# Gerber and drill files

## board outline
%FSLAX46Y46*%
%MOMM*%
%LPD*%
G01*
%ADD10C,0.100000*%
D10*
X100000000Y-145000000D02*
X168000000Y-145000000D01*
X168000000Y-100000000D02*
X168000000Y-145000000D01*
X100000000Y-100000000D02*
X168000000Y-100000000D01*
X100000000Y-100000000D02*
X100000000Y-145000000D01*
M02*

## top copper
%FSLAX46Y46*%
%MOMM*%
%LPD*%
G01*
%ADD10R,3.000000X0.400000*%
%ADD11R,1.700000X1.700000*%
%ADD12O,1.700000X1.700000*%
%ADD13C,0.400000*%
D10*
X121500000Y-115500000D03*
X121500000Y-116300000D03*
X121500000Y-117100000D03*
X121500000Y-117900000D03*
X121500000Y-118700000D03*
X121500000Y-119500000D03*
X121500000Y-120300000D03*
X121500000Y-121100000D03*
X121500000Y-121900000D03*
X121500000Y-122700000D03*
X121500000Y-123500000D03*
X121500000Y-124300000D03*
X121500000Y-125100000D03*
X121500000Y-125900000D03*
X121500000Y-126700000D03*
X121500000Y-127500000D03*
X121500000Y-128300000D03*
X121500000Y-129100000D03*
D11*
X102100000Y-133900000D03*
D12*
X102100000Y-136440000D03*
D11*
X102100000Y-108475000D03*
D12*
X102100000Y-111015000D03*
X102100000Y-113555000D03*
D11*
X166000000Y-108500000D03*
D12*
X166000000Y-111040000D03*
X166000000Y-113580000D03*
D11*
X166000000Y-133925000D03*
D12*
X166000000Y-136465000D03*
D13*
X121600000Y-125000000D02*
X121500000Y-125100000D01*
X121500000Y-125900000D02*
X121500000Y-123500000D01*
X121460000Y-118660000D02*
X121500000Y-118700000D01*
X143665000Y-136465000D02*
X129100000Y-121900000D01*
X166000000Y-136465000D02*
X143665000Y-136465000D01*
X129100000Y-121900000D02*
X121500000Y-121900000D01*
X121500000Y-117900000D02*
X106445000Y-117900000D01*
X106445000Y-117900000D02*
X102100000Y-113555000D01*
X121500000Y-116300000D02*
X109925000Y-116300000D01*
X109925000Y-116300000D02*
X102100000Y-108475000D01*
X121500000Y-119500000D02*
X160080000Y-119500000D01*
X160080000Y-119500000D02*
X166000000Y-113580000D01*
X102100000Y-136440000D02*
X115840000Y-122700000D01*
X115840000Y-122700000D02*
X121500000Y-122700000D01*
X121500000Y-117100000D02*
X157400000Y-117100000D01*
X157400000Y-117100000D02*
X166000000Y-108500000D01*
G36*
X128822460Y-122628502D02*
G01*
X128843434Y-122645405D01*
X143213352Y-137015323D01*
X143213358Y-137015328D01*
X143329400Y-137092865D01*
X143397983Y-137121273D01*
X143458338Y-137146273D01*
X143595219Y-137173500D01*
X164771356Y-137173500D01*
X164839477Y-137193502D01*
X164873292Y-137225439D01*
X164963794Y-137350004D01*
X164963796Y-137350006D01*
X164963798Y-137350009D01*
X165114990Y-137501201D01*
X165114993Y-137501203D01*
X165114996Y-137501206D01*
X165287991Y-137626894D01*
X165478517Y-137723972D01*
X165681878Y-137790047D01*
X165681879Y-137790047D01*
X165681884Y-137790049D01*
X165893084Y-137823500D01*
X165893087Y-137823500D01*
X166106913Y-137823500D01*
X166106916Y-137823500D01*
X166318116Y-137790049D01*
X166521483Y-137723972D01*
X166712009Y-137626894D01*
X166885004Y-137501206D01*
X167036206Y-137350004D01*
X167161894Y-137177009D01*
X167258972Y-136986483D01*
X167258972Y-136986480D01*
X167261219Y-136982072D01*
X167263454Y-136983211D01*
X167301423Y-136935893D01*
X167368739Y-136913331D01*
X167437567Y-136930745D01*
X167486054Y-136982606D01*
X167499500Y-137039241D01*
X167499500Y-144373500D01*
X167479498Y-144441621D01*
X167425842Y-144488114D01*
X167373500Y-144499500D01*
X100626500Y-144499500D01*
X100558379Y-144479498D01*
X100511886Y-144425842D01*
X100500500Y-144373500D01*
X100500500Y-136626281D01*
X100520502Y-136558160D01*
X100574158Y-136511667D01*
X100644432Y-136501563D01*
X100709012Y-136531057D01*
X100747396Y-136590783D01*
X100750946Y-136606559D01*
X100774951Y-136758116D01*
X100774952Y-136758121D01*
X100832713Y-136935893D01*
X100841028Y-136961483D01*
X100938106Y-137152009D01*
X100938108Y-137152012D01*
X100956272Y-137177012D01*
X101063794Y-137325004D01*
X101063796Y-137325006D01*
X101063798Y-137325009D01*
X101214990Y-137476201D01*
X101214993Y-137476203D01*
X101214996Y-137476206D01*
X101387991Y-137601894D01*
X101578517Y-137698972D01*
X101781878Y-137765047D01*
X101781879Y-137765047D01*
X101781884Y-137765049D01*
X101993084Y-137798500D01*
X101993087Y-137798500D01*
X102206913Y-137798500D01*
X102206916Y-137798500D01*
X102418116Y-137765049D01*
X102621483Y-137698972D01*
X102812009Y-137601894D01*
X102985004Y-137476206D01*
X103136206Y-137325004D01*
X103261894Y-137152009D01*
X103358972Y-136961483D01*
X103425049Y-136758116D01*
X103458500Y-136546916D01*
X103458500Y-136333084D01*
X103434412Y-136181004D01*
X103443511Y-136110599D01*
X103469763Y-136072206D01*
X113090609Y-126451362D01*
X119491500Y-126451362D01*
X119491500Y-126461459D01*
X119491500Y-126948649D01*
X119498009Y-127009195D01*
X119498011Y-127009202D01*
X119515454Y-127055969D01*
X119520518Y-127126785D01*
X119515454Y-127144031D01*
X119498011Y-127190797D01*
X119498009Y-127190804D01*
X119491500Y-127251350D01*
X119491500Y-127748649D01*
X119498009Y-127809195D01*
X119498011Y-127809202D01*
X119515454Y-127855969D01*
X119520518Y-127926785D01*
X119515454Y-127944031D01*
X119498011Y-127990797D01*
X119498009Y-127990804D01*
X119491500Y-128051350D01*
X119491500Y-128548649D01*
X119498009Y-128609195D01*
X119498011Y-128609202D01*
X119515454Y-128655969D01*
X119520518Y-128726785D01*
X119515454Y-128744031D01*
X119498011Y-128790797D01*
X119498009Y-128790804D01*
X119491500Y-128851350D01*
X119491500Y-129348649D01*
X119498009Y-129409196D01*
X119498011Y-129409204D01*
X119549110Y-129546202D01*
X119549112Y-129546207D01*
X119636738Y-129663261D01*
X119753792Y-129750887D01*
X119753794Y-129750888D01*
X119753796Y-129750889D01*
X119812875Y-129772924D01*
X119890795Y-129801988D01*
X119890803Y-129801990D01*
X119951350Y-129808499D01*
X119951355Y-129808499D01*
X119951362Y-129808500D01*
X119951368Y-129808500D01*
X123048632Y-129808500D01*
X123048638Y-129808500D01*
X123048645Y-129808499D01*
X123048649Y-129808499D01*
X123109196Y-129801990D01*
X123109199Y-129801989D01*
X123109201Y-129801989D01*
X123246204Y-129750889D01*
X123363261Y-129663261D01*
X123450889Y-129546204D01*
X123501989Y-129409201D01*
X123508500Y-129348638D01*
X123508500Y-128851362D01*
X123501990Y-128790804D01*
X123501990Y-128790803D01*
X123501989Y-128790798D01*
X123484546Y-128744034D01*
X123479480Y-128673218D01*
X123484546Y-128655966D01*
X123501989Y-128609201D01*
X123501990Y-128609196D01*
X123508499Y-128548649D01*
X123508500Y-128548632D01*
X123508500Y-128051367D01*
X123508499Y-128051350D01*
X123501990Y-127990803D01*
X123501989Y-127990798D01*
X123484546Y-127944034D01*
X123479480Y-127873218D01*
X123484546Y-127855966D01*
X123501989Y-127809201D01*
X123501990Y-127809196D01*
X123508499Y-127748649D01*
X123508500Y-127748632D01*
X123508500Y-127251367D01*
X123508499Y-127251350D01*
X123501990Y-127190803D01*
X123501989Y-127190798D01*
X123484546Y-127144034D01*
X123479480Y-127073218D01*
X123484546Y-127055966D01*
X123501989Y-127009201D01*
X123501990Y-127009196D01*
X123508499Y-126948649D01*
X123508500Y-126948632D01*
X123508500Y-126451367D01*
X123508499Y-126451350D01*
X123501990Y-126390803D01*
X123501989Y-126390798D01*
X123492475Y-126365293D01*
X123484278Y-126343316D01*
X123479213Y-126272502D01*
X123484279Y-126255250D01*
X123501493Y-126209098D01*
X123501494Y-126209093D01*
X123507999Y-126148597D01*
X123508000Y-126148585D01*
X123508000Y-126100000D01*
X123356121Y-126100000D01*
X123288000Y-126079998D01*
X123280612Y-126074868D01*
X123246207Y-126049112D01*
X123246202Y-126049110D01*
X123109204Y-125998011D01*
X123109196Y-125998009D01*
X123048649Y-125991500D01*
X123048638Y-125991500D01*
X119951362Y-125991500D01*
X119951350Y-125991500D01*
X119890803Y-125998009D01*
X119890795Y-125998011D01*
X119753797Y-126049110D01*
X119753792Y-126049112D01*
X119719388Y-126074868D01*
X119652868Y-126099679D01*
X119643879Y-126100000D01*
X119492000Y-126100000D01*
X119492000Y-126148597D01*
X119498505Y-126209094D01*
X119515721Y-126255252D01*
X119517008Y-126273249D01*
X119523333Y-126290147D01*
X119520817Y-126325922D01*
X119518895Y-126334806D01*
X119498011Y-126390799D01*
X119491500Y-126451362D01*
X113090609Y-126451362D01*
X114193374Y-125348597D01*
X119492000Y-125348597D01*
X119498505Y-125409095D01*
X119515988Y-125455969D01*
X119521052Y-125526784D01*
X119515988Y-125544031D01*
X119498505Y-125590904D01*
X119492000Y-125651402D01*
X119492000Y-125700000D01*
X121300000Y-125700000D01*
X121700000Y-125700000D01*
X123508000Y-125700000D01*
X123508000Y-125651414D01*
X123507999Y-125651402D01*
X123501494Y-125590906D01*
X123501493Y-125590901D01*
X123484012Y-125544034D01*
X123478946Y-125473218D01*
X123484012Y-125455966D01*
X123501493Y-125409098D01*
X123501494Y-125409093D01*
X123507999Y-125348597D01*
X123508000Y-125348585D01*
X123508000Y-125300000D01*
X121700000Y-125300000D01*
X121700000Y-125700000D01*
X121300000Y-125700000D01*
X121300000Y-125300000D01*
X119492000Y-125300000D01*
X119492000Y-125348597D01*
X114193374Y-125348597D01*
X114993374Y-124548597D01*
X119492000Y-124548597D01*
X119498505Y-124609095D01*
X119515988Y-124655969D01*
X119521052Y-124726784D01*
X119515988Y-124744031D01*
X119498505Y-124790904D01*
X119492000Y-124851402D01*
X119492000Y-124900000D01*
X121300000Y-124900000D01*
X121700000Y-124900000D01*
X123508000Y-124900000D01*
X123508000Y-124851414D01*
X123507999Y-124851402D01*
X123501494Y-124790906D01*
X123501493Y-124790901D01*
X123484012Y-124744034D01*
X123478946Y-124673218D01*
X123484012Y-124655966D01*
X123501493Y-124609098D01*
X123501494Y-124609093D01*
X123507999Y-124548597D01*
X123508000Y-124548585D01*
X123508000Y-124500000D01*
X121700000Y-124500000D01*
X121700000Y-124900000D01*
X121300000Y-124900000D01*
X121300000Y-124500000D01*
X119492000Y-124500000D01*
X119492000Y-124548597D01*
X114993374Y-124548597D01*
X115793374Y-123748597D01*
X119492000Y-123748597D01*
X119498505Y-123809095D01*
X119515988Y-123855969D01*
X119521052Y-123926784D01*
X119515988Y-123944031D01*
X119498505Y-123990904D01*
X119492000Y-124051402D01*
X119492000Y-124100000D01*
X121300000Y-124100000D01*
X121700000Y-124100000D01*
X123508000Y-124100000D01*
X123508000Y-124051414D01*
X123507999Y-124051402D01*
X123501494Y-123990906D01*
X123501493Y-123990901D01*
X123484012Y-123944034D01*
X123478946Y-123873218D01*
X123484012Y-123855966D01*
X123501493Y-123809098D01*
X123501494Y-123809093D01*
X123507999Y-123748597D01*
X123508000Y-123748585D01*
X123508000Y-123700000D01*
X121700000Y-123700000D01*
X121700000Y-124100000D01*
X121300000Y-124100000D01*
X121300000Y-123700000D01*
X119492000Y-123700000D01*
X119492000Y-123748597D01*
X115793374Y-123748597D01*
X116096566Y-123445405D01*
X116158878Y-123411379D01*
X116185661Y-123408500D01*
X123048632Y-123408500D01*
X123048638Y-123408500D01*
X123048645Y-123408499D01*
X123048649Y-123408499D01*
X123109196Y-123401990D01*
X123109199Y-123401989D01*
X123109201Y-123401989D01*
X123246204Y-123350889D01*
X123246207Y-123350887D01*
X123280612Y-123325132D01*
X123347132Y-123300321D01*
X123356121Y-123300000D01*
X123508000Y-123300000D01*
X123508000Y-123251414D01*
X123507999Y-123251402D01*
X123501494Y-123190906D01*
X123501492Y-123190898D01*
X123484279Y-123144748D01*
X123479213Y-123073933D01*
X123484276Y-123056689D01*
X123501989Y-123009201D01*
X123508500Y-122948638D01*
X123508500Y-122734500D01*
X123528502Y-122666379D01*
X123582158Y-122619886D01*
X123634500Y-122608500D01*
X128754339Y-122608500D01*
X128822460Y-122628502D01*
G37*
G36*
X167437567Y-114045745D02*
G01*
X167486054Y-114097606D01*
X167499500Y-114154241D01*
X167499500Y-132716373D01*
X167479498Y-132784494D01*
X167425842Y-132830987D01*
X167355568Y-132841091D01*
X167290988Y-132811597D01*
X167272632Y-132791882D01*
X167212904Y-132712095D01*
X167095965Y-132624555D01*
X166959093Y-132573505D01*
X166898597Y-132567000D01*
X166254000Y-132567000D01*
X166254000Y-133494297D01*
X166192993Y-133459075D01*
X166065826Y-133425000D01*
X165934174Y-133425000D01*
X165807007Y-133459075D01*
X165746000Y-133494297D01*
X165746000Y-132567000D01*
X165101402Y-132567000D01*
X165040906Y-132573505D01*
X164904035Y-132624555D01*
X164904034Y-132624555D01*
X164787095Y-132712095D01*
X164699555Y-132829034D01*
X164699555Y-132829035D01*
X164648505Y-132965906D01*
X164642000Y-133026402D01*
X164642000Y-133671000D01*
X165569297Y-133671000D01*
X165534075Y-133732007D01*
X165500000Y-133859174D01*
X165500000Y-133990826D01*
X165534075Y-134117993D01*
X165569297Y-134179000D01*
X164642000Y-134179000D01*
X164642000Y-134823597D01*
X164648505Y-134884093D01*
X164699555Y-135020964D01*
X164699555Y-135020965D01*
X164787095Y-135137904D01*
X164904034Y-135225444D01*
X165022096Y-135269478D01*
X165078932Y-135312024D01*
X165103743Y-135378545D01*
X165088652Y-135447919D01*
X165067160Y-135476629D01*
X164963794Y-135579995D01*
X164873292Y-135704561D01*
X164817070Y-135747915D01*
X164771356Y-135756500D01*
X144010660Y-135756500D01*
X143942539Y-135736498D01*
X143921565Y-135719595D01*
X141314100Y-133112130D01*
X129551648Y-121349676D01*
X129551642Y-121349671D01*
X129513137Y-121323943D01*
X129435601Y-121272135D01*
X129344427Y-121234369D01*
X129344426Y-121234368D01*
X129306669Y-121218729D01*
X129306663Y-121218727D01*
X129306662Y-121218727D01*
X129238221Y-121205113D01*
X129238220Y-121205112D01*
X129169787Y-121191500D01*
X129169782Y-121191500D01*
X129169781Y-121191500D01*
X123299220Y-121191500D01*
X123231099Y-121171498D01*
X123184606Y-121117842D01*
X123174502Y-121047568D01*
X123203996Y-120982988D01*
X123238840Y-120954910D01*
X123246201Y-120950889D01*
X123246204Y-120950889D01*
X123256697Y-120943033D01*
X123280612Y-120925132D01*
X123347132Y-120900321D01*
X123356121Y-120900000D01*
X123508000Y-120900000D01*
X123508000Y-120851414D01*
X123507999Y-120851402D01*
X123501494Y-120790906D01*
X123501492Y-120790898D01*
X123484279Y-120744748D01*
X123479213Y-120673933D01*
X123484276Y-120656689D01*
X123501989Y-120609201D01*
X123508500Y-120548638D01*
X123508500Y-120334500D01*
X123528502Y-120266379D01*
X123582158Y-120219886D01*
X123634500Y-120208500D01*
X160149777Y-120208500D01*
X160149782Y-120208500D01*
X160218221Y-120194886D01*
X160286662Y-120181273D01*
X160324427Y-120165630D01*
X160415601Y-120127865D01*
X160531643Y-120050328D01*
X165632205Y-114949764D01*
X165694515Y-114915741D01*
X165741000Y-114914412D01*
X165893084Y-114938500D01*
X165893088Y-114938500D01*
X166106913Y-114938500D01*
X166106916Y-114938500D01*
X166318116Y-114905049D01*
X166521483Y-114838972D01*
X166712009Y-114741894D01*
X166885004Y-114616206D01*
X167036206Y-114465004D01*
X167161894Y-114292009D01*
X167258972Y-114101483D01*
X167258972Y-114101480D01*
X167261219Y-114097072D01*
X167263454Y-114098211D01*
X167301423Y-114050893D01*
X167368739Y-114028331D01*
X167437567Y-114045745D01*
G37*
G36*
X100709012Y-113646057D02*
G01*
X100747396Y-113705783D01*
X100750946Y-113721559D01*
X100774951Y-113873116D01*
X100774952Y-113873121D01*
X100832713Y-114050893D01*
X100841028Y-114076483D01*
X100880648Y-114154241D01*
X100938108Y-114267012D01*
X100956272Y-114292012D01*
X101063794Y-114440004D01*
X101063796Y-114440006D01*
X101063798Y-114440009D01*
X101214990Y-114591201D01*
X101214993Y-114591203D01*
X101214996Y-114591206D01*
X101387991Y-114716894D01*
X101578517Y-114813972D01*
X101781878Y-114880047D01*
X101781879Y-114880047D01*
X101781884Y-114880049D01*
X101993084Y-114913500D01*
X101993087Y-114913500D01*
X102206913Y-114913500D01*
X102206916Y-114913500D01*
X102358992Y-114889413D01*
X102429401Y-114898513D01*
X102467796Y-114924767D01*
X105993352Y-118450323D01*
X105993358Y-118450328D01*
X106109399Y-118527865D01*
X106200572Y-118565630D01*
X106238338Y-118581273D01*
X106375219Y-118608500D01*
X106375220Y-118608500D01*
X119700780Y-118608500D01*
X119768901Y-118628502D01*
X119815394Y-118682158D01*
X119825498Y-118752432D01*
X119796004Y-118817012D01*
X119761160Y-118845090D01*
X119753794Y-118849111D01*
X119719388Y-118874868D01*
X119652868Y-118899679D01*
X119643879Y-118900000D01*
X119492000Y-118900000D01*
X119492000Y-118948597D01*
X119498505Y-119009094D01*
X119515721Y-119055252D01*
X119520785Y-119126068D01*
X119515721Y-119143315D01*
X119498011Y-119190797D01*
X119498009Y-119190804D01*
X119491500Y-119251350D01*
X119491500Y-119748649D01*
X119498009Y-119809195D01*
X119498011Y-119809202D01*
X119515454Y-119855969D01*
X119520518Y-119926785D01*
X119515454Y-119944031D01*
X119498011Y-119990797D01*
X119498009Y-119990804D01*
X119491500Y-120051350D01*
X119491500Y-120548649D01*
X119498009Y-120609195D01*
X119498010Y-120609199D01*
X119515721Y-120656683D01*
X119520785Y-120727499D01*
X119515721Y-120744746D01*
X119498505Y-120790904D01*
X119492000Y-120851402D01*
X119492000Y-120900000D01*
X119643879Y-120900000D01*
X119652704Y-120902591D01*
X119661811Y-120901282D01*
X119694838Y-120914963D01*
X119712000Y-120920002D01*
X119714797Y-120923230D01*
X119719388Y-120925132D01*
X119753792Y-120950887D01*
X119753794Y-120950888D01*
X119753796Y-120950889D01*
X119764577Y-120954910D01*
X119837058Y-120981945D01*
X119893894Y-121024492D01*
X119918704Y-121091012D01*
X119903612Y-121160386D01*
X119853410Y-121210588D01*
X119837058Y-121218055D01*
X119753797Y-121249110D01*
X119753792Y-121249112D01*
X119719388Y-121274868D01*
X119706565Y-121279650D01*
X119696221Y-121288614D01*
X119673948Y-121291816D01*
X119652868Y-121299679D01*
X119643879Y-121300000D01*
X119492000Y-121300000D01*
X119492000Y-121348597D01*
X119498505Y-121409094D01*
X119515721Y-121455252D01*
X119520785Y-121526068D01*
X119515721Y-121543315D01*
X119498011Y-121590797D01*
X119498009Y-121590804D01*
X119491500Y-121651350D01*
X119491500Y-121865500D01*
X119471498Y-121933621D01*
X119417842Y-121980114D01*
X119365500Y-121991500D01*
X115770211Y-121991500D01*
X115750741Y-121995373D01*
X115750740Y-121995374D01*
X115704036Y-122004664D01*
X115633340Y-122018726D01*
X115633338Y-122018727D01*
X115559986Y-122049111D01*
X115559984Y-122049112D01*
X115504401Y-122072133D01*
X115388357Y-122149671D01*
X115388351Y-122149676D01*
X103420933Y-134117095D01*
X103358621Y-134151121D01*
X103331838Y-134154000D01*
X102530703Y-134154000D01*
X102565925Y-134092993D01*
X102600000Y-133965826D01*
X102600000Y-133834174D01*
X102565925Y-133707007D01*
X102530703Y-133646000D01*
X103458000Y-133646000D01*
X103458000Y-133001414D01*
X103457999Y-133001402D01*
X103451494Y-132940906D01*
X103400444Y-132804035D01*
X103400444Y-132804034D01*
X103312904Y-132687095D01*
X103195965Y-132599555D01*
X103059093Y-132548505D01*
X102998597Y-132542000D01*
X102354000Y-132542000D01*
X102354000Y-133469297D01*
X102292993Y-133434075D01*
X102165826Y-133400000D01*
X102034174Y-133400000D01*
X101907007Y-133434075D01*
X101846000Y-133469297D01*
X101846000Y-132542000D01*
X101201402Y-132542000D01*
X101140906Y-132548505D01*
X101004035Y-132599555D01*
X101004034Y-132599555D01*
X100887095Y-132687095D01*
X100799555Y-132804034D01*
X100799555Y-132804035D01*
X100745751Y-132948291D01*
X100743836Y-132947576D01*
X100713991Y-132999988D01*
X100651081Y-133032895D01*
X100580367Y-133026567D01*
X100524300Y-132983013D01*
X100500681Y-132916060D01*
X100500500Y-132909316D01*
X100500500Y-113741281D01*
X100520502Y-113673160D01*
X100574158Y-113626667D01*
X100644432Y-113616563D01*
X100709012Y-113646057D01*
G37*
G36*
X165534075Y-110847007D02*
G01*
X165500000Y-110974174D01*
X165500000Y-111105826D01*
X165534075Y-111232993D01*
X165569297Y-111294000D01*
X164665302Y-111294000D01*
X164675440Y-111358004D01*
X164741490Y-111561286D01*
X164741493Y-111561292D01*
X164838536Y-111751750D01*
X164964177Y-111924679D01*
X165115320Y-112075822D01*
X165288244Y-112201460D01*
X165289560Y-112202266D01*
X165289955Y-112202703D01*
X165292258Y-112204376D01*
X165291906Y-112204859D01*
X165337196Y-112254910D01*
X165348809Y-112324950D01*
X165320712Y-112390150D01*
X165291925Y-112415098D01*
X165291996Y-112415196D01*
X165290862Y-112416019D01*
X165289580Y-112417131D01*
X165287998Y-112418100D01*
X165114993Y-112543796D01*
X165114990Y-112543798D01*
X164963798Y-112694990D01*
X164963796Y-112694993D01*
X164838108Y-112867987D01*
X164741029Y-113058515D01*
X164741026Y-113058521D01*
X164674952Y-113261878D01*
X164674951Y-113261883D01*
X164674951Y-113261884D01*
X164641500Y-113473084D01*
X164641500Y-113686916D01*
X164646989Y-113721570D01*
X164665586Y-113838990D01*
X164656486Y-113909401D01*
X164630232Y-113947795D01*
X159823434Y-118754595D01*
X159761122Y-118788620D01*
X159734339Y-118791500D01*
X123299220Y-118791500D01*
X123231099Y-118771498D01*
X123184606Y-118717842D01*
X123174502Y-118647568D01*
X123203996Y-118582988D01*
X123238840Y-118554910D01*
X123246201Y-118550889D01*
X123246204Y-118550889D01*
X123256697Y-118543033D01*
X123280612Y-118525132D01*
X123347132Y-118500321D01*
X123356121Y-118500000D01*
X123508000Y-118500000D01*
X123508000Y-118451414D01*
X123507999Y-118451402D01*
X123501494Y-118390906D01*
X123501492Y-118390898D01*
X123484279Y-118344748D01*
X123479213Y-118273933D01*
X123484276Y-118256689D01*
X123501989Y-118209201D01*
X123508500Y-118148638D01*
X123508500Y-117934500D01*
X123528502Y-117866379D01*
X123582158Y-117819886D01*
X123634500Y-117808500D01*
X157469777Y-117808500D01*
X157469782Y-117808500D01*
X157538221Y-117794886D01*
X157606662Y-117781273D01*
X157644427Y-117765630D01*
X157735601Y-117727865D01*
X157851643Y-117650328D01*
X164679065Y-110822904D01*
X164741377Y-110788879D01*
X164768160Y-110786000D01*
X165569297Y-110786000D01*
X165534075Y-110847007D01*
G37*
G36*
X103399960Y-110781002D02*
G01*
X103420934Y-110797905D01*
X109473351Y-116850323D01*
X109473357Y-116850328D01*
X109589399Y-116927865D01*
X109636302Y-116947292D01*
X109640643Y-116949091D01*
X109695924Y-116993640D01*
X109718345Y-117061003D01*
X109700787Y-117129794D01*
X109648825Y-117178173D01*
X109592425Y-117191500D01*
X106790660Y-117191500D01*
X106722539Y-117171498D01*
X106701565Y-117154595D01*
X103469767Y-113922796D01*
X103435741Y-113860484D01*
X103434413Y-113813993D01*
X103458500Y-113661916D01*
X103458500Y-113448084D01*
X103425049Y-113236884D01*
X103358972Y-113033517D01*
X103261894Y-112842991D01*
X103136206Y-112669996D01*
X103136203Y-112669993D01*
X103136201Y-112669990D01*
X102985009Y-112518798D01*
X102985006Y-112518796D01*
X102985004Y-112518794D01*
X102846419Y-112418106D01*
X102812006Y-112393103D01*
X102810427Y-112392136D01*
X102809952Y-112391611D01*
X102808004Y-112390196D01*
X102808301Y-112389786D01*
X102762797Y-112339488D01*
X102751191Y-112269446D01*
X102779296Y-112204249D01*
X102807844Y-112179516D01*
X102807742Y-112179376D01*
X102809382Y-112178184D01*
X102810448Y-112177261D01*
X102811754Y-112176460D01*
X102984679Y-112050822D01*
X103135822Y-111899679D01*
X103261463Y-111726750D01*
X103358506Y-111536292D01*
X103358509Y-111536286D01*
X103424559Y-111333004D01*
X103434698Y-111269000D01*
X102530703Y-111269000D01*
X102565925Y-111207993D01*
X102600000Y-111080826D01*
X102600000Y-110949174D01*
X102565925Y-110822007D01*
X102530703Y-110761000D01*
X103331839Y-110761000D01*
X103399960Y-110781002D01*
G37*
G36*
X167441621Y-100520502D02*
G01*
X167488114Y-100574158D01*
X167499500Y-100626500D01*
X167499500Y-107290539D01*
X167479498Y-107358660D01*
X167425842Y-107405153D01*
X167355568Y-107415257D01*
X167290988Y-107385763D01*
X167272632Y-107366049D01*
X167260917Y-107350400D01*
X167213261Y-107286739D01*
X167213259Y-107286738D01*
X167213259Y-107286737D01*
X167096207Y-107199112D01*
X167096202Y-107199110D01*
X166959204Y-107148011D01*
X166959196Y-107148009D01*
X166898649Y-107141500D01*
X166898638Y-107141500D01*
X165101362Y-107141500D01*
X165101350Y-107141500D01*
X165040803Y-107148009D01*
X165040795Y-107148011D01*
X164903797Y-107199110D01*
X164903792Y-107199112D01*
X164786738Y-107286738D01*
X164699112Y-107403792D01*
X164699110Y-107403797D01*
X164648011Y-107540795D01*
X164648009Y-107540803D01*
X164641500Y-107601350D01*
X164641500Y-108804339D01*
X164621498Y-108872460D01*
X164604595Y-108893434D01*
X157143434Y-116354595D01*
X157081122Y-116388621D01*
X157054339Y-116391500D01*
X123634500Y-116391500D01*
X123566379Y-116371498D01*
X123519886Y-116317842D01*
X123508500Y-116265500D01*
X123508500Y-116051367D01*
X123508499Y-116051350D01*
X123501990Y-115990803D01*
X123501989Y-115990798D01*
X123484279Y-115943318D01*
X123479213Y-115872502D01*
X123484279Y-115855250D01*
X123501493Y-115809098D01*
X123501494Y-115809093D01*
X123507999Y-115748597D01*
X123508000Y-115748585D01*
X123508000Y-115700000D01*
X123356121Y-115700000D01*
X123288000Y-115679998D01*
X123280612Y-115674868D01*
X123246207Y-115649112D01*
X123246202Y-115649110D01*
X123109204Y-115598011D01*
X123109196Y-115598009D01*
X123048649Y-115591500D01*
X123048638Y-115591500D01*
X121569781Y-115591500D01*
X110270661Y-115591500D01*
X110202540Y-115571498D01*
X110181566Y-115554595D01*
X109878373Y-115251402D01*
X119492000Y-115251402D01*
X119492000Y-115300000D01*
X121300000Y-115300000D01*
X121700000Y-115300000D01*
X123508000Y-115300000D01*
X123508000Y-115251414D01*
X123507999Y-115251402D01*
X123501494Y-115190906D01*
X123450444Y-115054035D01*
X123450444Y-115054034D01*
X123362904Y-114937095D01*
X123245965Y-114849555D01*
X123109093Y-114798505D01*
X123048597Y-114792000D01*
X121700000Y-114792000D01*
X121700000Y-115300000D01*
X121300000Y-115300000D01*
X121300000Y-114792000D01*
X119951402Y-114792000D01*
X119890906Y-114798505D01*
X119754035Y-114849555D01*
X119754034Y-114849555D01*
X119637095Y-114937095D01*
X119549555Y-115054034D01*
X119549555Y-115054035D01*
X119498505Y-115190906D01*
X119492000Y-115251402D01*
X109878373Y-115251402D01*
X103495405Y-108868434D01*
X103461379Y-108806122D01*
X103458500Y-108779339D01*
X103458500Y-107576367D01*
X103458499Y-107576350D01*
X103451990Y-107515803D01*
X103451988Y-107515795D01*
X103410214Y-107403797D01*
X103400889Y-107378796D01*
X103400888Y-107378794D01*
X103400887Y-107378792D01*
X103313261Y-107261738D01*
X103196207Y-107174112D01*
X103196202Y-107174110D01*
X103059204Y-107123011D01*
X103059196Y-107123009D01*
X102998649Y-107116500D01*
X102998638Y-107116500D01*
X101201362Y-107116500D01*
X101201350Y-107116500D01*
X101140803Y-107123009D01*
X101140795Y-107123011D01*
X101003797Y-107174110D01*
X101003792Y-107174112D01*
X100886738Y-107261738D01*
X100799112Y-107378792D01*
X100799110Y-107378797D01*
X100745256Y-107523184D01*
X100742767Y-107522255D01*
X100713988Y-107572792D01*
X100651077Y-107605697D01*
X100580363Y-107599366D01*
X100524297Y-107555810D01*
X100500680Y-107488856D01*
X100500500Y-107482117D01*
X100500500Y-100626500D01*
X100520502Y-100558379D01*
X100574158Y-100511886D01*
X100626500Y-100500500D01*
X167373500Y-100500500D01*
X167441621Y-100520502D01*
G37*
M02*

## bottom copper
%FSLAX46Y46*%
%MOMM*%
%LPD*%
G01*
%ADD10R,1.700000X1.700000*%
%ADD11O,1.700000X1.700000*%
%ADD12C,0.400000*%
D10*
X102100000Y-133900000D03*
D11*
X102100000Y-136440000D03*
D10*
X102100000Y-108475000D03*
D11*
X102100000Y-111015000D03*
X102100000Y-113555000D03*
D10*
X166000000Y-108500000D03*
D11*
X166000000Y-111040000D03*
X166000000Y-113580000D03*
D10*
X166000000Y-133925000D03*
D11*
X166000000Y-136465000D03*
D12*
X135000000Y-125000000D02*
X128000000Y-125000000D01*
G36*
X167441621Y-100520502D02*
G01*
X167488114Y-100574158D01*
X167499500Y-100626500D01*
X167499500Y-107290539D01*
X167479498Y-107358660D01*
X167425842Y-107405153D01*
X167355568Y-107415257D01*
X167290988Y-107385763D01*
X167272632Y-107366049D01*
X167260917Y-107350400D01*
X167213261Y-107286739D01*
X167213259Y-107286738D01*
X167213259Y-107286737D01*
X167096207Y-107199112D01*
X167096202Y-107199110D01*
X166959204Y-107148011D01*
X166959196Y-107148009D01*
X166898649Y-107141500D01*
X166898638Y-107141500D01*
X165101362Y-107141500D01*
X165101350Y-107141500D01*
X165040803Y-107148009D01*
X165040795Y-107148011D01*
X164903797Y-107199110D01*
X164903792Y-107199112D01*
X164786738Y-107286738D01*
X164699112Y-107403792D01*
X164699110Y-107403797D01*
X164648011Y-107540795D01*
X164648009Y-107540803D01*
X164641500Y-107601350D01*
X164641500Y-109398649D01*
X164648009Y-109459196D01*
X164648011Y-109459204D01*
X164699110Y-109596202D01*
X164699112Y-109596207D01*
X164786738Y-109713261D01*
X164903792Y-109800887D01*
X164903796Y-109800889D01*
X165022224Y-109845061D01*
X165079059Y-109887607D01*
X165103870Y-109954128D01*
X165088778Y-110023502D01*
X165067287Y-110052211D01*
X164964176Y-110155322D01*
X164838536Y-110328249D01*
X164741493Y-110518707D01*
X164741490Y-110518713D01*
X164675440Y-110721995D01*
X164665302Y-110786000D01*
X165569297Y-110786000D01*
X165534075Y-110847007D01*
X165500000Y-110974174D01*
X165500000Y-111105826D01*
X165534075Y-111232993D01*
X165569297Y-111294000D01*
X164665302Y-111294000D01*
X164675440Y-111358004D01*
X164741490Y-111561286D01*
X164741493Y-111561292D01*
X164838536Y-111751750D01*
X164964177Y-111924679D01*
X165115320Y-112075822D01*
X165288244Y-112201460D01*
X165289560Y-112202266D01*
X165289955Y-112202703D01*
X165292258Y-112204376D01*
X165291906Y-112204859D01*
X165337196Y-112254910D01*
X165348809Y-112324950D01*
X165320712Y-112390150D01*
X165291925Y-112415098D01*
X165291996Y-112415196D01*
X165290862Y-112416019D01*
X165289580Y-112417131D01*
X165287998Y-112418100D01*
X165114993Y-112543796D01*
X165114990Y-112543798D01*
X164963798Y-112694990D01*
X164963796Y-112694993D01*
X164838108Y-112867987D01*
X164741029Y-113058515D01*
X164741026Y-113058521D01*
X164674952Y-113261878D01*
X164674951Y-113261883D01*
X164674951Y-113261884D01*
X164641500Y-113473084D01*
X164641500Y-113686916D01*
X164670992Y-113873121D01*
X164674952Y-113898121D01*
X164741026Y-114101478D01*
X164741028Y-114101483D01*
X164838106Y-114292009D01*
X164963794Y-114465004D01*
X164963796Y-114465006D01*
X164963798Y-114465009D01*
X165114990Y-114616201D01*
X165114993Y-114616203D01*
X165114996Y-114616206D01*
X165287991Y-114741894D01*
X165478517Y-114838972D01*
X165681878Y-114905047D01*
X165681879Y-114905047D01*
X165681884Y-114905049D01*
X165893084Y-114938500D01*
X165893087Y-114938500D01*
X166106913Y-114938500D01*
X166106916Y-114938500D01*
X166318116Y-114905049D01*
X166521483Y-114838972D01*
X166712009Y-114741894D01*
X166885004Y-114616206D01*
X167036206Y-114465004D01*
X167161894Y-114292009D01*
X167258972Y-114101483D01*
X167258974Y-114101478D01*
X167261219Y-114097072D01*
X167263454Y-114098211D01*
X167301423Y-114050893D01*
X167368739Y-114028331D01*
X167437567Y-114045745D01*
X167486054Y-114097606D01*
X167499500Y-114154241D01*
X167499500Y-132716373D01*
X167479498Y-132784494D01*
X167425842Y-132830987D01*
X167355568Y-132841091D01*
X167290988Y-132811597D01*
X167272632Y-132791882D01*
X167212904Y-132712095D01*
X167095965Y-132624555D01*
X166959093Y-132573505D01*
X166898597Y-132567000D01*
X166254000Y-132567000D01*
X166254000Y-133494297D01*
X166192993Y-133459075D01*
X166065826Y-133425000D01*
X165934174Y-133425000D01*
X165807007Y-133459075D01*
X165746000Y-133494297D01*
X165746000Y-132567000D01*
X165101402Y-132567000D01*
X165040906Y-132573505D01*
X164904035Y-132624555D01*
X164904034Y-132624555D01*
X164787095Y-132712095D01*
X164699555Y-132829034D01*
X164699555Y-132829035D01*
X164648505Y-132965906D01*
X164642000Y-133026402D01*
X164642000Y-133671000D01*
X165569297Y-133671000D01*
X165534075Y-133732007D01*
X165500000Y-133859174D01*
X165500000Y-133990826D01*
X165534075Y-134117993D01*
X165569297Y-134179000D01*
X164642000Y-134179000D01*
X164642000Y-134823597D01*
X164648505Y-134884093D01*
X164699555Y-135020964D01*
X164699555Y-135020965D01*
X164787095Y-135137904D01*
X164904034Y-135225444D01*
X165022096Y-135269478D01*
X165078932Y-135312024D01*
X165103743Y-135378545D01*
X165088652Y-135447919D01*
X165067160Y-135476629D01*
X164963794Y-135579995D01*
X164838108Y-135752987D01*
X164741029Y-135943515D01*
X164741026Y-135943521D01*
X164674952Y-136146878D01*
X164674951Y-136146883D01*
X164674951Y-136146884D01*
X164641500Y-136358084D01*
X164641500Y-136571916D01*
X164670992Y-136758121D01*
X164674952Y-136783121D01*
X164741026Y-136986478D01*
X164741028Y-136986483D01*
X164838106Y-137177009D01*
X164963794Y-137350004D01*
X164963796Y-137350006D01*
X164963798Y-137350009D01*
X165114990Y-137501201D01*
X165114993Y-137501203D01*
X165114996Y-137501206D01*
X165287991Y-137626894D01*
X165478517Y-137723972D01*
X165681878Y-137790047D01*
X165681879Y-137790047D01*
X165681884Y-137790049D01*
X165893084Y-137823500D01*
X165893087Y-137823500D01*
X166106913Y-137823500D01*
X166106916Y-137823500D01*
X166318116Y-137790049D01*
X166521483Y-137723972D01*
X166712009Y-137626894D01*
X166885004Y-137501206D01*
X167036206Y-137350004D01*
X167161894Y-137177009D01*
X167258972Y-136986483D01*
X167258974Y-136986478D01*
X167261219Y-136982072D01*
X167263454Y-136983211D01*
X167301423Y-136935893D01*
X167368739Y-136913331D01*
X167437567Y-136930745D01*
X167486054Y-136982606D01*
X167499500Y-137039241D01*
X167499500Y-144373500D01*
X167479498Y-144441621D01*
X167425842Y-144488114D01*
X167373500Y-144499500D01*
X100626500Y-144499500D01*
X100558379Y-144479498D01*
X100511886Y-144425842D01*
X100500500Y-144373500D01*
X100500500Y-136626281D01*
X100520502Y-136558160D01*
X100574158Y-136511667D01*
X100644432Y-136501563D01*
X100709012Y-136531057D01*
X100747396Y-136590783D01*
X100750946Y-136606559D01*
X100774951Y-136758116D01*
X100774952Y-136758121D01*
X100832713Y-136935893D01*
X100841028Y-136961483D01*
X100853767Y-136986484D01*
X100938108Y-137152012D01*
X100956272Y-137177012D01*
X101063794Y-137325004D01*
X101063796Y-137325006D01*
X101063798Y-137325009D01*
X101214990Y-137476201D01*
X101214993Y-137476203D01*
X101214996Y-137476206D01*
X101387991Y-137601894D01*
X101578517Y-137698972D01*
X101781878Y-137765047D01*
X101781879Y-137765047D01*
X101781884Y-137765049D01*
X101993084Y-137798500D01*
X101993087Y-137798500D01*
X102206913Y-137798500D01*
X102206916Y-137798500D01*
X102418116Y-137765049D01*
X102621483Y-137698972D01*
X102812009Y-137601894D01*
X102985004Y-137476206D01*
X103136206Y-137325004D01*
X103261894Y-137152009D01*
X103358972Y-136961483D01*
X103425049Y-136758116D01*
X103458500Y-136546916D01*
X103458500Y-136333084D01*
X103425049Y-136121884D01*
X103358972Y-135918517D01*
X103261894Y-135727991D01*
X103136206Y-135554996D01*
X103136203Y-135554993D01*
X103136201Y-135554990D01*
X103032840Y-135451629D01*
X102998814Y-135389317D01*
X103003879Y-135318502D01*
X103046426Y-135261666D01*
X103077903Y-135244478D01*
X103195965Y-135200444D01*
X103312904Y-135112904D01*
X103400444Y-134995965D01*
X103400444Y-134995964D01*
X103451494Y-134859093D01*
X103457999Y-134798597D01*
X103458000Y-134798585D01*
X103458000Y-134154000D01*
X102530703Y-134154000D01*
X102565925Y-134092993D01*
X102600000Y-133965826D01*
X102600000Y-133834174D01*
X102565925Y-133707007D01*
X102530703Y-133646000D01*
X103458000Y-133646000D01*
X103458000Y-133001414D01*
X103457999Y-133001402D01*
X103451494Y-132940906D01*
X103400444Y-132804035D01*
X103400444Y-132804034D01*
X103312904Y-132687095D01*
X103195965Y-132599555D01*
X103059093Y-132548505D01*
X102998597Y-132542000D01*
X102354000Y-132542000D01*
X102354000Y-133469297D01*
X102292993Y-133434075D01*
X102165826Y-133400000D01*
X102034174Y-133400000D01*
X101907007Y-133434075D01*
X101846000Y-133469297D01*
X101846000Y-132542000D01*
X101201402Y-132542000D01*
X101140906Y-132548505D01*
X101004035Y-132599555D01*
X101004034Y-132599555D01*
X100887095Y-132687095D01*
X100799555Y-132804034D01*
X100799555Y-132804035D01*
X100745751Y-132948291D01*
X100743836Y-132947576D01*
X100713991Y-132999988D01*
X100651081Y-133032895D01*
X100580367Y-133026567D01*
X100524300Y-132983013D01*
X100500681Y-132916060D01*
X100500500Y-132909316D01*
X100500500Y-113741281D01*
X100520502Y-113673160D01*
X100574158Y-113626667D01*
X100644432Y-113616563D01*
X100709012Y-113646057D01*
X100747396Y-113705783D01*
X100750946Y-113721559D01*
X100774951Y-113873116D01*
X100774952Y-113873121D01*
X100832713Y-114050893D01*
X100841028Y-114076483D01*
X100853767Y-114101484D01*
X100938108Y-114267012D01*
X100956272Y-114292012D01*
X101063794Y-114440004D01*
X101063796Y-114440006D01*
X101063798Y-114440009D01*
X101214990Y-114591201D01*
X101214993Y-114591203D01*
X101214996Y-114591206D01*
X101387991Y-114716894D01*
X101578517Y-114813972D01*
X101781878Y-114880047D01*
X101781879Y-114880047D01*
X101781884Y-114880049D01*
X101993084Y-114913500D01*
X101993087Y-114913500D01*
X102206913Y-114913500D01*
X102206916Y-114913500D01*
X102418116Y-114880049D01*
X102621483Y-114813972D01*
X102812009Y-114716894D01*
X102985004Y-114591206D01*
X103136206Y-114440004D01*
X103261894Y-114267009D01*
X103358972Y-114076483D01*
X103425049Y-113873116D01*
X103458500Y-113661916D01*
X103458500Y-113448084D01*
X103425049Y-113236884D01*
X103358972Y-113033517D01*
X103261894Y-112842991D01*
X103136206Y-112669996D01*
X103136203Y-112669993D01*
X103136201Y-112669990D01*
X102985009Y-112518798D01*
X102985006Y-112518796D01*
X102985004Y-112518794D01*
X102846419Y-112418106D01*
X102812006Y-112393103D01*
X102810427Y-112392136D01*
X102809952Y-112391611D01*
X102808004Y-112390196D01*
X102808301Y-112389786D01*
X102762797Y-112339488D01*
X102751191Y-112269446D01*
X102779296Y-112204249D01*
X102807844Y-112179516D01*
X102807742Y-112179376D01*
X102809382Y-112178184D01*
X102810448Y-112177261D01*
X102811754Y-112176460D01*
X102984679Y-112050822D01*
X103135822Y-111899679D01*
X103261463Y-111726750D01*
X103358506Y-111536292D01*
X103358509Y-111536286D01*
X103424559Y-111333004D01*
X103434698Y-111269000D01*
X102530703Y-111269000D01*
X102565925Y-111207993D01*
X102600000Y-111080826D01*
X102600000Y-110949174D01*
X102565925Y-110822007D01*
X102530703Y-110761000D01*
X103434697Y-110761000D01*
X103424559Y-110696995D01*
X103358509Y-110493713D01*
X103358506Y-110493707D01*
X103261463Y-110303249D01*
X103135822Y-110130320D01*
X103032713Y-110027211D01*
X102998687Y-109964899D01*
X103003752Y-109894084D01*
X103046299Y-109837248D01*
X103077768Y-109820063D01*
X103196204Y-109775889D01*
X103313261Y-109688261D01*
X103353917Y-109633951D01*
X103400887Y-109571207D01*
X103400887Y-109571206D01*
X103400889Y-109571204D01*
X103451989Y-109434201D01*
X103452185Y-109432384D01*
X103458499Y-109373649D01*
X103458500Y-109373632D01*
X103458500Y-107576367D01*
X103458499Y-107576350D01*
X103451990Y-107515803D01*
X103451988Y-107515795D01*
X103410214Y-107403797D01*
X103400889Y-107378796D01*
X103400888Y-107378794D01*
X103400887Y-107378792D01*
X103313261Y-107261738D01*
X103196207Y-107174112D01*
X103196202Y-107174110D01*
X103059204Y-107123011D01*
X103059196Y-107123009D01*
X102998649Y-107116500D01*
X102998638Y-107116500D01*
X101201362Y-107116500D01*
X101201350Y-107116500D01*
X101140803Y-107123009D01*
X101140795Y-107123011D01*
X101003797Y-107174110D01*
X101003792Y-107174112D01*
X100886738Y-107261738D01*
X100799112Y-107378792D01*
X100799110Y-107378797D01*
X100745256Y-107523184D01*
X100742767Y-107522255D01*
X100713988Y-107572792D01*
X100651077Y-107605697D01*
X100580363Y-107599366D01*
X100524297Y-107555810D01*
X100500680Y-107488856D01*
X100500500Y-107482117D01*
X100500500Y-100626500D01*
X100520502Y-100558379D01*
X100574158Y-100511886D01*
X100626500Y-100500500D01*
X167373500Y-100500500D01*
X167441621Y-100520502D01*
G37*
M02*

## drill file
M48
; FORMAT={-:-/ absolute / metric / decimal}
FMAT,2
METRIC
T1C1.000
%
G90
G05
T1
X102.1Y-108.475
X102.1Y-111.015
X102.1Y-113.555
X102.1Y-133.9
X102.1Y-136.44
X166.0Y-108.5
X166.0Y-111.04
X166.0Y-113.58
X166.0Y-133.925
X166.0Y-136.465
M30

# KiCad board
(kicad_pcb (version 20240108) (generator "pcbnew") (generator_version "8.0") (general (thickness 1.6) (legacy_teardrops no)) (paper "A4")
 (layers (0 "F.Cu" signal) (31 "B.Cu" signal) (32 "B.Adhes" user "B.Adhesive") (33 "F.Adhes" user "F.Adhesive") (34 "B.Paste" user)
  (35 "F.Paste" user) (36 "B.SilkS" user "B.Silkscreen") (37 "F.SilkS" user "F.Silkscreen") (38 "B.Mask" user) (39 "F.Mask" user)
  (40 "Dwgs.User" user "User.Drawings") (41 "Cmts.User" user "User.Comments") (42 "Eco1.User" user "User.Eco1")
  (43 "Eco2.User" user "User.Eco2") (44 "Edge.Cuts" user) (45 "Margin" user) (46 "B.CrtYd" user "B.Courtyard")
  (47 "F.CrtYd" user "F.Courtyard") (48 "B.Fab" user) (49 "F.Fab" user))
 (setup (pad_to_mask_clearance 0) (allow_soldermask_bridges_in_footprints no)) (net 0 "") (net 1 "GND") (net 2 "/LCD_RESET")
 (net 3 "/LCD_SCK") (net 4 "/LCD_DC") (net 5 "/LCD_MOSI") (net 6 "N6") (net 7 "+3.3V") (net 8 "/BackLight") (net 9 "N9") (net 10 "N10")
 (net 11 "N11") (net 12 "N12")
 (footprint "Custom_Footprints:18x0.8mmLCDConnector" (layer "F.Cu") (at 121.5 115.5 -90)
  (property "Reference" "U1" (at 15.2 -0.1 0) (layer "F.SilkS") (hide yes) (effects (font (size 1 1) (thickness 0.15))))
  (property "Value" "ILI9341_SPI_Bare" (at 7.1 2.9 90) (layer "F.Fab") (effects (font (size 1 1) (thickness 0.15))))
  (pad "1" smd rect (at 0 0 270) (size 0.4 3) (layers "F.Cu" "F.Paste" "F.Mask") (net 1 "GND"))
  (pad "2" smd rect (at 0.8 0 270) (size 0.4 3) (layers "F.Cu" "F.Paste" "F.Mask") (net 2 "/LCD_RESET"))
  (pad "3" smd rect (at 1.6 0 270) (size 0.4 3) (layers "F.Cu" "F.Paste" "F.Mask") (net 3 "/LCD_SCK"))
  (pad "4" smd rect (at 2.4 0 270) (size 0.4 3) (layers "F.Cu" "F.Paste" "F.Mask") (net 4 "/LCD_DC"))
  (pad "5" smd rect (at 3.2 0 270) (size 0.4 3) (layers "F.Cu" "F.Paste" "F.Mask") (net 1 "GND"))
  (pad "6" smd rect (at 4 0 270) (size 0.4 3) (layers "F.Cu" "F.Paste" "F.Mask") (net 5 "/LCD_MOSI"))
  (pad "7" smd rect (at 4.8 0 270) (size 0.4 3) (layers "F.Cu" "F.Paste" "F.Mask") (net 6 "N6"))
  (pad "8" smd rect (at 5.6 0 270) (size 0.4 3) (layers "F.Cu" "F.Paste" "F.Mask") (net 1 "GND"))
  (pad "9" smd rect (at 6.4 0 270) (size 0.4 3) (layers "F.Cu" "F.Paste" "F.Mask") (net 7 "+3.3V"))
  (pad "10" smd rect (at 7.2 0 270) (size 0.4 3) (layers "F.Cu" "F.Paste" "F.Mask") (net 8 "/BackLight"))
  (pad "11" smd rect (at 8 0 270) (size 0.4 3) (layers "F.Cu" "F.Paste" "F.Mask") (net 1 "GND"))
  (pad "12" smd rect (at 8.8 0 270) (size 0.4 3) (layers "F.Cu" "F.Paste" "F.Mask") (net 1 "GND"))
  (pad "13" smd rect (at 9.6 0 270) (size 0.4 3) (layers "F.Cu" "F.Paste" "F.Mask") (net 1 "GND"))
  (pad "14" smd rect (at 10.4 0 270) (size 0.4 3) (layers "F.Cu" "F.Paste" "F.Mask") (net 1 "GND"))
  (pad "15" smd rect (at 11.2 0 270) (size 0.4 3) (layers "F.Cu" "F.Paste" "F.Mask") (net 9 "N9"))
  (pad "16" smd rect (at 12 0 270) (size 0.4 3) (layers "F.Cu" "F.Paste" "F.Mask") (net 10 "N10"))
  (pad "17" smd rect (at 12.8 0 270) (size 0.4 3) (layers "F.Cu" "F.Paste" "F.Mask") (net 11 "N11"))
  (pad "18" smd rect (at 13.6 0 270) (size 0.4 3) (layers "F.Cu" "F.Paste" "F.Mask") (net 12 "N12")))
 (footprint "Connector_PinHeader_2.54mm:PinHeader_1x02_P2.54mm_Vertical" (layer "F.Cu") (at 102.1 133.9)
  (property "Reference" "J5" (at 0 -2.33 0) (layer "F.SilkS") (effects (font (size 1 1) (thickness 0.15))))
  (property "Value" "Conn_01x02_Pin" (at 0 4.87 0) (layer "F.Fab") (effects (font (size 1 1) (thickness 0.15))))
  (pad "1" thru_hole rect (at 0 0) (size 1.7 1.7) (drill 1) (layers "*.Cu" "*.Mask") (remove_unused_layers no) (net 1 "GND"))
  (pad "2" thru_hole oval (at 0 2.54) (size 1.7 1.7) (drill 1) (layers "*.Cu" "*.Mask") (remove_unused_layers no) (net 8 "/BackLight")))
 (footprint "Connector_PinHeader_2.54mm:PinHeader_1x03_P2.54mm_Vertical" (layer "F.Cu") (at 102.1 108.475)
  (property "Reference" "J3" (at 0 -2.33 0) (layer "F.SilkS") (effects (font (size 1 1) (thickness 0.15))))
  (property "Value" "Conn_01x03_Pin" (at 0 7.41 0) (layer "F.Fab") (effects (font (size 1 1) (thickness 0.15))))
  (pad "1" thru_hole rect (at 0 0) (size 1.7 1.7) (drill 1) (layers "*.Cu" "*.Mask") (remove_unused_layers no) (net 2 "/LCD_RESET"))
  (pad "2" thru_hole oval (at 0 2.54) (size 1.7 1.7) (drill 1) (layers "*.Cu" "*.Mask") (remove_unused_layers no) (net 1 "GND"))
  (pad "3" thru_hole oval (at 0 5.08) (size 1.7 1.7) (drill 1) (layers "*.Cu" "*.Mask") (remove_unused_layers no) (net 4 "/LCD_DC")))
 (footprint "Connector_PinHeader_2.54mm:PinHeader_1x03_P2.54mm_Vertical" (layer "F.Cu") (at 166 108.5)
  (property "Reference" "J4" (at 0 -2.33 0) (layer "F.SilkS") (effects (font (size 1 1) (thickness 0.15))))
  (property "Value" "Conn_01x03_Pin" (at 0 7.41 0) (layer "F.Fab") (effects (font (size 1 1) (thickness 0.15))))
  (pad "1" thru_hole rect (at 0 0) (size 1.7 1.7) (drill 1) (layers "*.Cu" "*.Mask") (remove_unused_layers no) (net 3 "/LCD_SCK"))
  (pad "2" thru_hole oval (at 0 2.54) (size 1.7 1.7) (drill 1) (layers "*.Cu" "*.Mask") (remove_unused_layers no) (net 1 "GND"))
  (pad "3" thru_hole oval (at 0 5.08) (size 1.7 1.7) (drill 1) (layers "*.Cu" "*.Mask") (remove_unused_layers no) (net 5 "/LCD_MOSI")))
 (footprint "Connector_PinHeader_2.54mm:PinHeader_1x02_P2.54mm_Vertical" (layer "F.Cu") (at 166 133.925)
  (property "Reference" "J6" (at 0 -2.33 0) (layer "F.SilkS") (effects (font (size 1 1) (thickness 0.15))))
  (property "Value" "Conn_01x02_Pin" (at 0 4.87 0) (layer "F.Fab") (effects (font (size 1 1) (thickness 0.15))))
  (pad "1" thru_hole rect (at 0 0) (size 1.7 1.7) (drill 1) (layers "*.Cu" "*.Mask") (remove_unused_layers no) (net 1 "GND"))
  (pad "2" thru_hole oval (at 0 2.54) (size 1.7 1.7) (drill 1) (layers "*.Cu" "*.Mask") (remove_unused_layers no) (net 7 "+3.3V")))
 (gr_line (start 100 145) (end 168 145) (stroke (width 0.1) (type solid)) (layer "Edge.Cuts"))
 (gr_line (start 168 100) (end 168 145) (stroke (width 0.1) (type solid)) (layer "Edge.Cuts"))
 (gr_line (start 100 100) (end 168 100) (stroke (width 0.1) (type solid)) (layer "Edge.Cuts"))
 (gr_line (start 100 100) (end 100 145) (stroke (width 0.1) (type solid)) (layer "Edge.Cuts"))
 (segment (start 121.6 125) (end 121.5 125.1) (width 0.4) (layer "F.Cu") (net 1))
 (segment (start 121.5 125.9) (end 121.5 123.5) (width 0.4) (layer "F.Cu") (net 1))
 (segment (start 121.46 118.66) (end 121.5 118.7) (width 0.4) (layer "F.Cu") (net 1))
 (segment (start 135 125) (end 128 125) (width 0.4) (layer "B.Cu") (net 1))
 (segment (start 143.665 136.465) (end 129.1 121.9) (width 0.4) (layer "F.Cu") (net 7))
 (segment (start 166 136.465) (end 143.665 136.465) (width 0.4) (layer "F.Cu") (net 7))
 (segment (start 129.1 121.9) (end 121.5 121.9) (width 0.4) (layer "F.Cu") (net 7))
 (segment (start 121.5 117.9) (end 106.445 117.9) (width 0.4) (layer "F.Cu") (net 4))
 (segment (start 106.445 117.9) (end 102.1 113.555) (width 0.4) (layer "F.Cu") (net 4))
 (segment (start 121.5 116.3) (end 109.925 116.3) (width 0.4) (layer "F.Cu") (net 2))
 (segment (start 109.925 116.3) (end 102.1 108.475) (width 0.4) (layer "F.Cu") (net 2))
 (segment (start 121.5 119.5) (end 160.08 119.5) (width 0.4) (layer "F.Cu") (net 5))
 (segment (start 160.08 119.5) (end 166 113.58) (width 0.4) (layer "F.Cu") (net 5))
 (segment (start 102.1 136.44) (end 115.84 122.7) (width 0.4) (layer "F.Cu") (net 8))
 (segment (start 115.84 122.7) (end 121.5 122.7) (width 0.4) (layer "F.Cu") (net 8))
 (segment (start 121.5 117.1) (end 157.4 117.1) (width 0.4) (layer "F.Cu") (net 3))
 (segment (start 157.4 117.1) (end 166 108.5) (width 0.4) (layer "F.Cu") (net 3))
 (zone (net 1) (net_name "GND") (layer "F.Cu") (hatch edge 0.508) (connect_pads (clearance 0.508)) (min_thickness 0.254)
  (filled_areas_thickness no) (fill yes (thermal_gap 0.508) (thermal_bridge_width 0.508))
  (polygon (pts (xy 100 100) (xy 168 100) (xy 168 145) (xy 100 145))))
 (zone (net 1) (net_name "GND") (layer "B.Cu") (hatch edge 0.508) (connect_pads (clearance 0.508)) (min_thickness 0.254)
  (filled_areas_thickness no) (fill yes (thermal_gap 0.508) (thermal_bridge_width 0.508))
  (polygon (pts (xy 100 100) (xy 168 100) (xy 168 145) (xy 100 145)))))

